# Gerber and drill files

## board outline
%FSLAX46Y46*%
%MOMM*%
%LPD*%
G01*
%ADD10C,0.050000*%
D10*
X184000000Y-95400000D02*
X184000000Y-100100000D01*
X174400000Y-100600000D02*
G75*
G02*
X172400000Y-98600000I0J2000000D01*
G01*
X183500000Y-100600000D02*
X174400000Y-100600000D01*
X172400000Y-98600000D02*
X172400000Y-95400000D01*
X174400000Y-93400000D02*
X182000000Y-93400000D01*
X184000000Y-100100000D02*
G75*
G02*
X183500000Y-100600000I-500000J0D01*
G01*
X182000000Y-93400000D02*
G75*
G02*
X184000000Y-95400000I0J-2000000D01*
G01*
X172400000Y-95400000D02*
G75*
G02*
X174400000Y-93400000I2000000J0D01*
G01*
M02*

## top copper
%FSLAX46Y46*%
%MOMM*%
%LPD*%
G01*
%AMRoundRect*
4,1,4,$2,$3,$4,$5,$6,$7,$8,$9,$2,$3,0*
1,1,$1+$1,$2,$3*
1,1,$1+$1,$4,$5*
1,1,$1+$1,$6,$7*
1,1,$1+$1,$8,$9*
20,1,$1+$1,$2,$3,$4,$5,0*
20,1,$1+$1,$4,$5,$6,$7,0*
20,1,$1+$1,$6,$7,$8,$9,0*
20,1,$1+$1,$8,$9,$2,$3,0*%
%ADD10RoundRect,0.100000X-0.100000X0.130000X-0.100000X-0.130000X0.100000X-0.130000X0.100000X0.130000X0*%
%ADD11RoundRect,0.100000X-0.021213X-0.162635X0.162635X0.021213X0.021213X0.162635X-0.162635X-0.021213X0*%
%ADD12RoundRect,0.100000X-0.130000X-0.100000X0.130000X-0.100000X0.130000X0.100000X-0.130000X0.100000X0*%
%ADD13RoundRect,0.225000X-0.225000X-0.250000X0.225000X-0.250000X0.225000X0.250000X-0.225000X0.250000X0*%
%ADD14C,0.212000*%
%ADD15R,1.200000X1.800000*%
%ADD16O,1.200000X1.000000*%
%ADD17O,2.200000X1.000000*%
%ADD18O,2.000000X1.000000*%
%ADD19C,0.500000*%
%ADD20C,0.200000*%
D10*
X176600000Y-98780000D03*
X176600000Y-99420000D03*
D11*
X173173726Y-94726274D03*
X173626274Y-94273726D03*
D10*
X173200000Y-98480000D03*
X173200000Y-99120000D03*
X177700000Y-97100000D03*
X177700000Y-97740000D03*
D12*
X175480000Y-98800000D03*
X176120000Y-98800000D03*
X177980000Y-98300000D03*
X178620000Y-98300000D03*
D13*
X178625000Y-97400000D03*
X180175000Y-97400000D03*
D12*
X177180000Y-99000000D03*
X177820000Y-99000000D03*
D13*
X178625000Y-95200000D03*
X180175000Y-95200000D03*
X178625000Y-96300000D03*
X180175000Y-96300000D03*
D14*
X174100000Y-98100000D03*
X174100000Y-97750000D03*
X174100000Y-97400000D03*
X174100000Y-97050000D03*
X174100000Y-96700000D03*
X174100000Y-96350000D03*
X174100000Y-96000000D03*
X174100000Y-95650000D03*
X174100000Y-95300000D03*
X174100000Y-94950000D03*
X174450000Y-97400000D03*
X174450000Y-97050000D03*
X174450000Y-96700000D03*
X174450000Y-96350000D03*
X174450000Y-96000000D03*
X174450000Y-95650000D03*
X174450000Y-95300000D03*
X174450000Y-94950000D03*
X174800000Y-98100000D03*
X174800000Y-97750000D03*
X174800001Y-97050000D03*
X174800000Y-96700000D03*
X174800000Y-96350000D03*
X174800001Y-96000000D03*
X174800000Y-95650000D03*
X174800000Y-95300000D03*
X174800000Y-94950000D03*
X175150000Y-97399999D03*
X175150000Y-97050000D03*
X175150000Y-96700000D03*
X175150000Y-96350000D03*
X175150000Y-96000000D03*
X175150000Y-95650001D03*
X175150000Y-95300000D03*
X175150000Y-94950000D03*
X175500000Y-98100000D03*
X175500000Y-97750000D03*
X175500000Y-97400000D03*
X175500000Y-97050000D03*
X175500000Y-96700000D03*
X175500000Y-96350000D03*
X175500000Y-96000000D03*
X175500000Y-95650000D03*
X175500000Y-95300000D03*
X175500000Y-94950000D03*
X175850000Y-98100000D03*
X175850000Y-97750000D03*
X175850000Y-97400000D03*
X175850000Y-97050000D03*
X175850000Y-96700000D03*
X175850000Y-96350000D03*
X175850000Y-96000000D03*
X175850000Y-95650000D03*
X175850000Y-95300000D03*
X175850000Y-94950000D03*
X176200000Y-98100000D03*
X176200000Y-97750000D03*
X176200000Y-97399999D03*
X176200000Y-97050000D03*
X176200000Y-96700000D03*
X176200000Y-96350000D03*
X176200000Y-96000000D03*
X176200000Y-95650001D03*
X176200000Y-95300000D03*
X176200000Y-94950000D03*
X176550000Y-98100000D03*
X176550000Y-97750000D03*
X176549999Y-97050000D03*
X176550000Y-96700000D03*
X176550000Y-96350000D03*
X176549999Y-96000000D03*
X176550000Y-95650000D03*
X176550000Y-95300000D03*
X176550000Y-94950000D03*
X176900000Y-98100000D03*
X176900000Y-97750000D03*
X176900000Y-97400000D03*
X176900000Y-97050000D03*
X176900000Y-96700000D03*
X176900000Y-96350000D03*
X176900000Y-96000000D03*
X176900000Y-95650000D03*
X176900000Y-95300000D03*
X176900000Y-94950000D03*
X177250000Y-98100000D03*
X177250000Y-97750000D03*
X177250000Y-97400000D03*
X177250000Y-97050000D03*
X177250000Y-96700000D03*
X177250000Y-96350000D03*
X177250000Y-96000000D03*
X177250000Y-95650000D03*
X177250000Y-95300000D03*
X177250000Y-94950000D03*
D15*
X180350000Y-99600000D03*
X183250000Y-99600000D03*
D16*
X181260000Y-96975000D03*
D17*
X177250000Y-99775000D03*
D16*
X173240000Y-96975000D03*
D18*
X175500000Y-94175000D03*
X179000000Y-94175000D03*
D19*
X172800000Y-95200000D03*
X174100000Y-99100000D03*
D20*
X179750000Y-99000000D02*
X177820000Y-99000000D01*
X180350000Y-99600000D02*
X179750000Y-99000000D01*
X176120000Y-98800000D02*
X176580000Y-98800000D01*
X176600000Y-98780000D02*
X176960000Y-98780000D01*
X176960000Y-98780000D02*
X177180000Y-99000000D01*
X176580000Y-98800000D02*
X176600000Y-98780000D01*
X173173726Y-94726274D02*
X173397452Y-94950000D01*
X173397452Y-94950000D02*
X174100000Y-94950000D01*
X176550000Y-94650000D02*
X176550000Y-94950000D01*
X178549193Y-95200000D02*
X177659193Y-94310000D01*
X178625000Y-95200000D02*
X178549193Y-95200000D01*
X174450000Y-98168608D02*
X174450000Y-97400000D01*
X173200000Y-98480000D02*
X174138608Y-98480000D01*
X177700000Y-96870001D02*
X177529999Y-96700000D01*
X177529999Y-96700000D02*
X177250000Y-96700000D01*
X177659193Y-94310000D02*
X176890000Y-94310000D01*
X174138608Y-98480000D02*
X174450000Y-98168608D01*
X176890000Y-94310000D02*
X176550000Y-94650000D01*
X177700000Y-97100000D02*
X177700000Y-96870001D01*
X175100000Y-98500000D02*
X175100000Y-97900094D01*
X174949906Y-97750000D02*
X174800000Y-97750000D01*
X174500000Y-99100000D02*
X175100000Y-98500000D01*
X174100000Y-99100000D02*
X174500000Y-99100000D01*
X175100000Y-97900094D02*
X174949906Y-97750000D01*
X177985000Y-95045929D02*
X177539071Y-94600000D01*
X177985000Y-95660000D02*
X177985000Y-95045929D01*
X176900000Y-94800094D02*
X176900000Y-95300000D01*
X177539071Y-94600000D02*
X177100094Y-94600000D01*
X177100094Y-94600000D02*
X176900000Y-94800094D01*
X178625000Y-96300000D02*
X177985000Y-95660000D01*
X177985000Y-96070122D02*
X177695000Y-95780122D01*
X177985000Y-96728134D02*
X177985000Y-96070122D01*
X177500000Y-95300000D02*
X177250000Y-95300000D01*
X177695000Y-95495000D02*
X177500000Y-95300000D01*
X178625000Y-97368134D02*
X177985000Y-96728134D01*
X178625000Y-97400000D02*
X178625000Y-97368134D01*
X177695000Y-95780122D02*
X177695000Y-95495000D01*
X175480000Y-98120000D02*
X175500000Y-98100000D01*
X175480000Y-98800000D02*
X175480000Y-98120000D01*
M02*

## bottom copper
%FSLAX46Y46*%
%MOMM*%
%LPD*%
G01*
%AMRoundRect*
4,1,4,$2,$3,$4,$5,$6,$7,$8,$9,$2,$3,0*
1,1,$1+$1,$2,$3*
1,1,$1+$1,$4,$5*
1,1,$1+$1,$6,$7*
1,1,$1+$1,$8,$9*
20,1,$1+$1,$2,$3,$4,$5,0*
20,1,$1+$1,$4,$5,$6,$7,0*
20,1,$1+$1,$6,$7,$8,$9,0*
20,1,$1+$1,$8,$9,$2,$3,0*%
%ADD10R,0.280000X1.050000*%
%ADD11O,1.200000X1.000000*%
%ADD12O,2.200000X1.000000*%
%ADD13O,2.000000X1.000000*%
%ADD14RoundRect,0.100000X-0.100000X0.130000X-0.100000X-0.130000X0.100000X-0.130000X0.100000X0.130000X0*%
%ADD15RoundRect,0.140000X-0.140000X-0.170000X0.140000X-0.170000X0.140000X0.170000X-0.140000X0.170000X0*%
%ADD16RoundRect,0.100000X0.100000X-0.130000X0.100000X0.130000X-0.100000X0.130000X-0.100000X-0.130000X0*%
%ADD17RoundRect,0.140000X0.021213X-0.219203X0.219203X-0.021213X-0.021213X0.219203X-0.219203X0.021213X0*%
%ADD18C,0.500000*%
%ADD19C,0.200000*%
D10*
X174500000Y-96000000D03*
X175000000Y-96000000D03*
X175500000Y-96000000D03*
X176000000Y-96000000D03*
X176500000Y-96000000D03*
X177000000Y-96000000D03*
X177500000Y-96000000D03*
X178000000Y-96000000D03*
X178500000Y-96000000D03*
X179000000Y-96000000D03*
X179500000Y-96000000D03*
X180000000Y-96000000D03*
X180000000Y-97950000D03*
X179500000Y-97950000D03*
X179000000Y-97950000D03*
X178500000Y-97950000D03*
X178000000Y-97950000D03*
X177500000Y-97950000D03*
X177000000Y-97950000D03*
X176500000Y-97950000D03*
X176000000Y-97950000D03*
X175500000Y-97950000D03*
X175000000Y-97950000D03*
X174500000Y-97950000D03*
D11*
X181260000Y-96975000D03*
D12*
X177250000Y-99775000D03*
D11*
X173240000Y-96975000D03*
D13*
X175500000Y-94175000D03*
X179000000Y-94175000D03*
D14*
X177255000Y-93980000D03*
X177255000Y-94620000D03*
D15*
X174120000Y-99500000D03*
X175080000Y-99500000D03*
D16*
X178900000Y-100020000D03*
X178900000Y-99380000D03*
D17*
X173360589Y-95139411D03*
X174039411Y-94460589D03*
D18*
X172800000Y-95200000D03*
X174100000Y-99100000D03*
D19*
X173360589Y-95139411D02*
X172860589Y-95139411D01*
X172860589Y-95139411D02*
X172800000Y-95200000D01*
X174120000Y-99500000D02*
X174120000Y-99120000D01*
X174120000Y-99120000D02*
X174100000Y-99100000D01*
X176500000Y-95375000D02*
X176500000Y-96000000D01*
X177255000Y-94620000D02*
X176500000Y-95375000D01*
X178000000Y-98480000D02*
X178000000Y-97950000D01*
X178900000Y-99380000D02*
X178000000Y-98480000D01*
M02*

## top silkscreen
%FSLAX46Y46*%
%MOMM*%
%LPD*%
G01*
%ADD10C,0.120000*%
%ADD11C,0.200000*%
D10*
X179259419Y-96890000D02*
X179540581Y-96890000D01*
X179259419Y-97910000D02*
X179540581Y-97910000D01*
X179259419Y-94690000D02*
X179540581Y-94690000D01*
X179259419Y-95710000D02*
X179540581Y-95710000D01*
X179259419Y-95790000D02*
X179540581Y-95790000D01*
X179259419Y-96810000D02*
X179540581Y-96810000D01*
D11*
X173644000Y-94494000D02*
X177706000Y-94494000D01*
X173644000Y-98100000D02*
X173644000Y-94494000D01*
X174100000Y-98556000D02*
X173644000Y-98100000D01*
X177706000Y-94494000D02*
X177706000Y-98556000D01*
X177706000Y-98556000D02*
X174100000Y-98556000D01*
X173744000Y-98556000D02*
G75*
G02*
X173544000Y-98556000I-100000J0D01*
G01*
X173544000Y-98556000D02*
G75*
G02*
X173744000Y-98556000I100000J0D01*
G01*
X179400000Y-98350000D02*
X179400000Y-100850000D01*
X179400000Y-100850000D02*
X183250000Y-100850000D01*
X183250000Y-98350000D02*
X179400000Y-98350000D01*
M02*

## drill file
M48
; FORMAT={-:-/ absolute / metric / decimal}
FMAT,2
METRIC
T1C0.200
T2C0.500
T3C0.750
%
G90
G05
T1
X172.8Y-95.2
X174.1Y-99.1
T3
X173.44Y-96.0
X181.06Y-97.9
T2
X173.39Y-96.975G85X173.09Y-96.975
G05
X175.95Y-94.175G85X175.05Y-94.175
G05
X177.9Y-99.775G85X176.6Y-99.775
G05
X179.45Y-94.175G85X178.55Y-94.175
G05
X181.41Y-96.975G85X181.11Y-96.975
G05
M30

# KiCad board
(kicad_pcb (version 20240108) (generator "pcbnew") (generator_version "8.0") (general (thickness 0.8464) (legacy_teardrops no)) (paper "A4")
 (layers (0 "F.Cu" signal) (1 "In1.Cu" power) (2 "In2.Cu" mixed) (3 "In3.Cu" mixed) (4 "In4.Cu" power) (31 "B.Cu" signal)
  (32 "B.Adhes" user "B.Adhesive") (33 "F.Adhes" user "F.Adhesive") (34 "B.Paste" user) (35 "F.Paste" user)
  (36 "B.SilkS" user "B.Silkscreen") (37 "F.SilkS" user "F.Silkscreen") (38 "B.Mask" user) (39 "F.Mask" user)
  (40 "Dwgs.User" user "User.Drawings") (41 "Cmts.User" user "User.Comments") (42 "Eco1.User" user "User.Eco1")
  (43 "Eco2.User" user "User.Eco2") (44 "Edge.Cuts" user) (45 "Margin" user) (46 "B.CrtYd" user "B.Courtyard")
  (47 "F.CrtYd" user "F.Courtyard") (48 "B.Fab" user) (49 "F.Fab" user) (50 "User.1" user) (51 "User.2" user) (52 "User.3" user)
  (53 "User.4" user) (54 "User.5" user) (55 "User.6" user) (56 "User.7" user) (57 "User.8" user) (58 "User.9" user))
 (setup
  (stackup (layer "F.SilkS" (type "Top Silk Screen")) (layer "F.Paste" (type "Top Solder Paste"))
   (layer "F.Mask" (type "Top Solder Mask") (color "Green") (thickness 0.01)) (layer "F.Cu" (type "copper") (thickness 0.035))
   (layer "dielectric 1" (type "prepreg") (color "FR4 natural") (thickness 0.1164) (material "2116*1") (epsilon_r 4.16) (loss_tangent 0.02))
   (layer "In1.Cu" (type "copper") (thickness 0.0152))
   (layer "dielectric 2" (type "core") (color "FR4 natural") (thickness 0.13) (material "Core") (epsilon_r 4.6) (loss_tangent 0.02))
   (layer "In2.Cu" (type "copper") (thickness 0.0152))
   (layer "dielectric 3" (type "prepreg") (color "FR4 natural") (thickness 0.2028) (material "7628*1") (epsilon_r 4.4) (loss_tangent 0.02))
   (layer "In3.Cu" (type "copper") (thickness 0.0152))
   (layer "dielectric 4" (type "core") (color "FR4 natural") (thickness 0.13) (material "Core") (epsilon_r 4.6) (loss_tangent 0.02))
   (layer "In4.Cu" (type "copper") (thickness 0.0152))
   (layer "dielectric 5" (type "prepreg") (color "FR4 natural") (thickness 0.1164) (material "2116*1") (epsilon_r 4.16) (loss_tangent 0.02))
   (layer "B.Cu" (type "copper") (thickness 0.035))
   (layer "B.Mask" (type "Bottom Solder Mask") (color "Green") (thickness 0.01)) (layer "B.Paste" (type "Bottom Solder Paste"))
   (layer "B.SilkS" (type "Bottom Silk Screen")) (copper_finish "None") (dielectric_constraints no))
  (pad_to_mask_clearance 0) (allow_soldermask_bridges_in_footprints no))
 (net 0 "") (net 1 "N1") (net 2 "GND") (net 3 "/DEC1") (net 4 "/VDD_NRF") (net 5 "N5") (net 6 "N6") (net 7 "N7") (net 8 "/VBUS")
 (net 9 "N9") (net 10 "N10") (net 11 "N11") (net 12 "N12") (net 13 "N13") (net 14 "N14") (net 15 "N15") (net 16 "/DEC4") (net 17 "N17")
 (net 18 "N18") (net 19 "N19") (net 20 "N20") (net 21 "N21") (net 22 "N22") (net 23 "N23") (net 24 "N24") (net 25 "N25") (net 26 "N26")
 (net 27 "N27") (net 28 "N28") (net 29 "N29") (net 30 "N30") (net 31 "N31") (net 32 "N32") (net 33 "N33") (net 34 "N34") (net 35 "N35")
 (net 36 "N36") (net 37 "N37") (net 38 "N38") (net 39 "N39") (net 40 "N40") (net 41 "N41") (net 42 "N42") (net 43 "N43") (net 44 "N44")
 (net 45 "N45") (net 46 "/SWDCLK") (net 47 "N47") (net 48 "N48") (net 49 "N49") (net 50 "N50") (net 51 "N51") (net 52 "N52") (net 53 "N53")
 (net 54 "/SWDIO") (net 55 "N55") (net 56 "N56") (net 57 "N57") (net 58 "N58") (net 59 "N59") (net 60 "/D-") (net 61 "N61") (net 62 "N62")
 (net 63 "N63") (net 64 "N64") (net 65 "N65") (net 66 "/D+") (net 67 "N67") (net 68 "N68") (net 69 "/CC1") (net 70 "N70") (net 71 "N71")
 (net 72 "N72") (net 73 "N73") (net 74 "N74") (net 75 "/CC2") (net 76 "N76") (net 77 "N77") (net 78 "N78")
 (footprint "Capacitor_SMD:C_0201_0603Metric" (layer "F.Cu") (at 176.6 99.1 -90)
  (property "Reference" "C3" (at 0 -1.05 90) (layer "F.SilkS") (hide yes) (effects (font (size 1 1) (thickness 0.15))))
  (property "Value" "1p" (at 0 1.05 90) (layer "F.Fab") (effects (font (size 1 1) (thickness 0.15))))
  (pad "" smd roundrect (at -0.345 0 270) (size 0.318 0.36) (layers "F.Paste") (roundrect_rratio 0.25))
  (pad "" smd roundrect (at 0.345 0 270) (size 0.318 0.36) (layers "F.Paste") (roundrect_rratio 0.25))
  (pad "1" smd roundrect (at -0.32 0 270) (size 0.46 0.4) (layers "F.Cu" "F.Mask") (roundrect_rratio 0.25) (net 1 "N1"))
  (pad "2" smd roundrect (at 0.32 0 270) (size 0.46 0.4) (layers "F.Cu" "F.Mask") (roundrect_rratio 0.25) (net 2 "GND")))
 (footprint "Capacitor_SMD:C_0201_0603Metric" (layer "F.Cu") (at 173.4 94.5 45)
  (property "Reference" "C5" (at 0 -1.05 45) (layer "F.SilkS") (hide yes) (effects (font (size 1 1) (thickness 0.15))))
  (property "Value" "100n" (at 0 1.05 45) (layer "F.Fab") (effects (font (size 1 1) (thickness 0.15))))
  (pad "" smd roundrect (at -0.345 0 45) (size 0.318 0.36) (layers "F.Paste") (roundrect_rratio 0.25))
  (pad "" smd roundrect (at 0.345 0 45) (size 0.318 0.36) (layers "F.Paste") (roundrect_rratio 0.25))
  (pad "1" smd roundrect (at -0.32 0 45) (size 0.46 0.4) (layers "F.Cu" "F.Mask") (roundrect_rratio 0.25) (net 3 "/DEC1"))
  (pad "2" smd roundrect (at 0.32 0 45) (size 0.46 0.4) (layers "F.Cu" "F.Mask") (roundrect_rratio 0.25) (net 2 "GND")))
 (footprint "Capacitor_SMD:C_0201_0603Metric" (layer "F.Cu") (at 173.2 98.8 -90)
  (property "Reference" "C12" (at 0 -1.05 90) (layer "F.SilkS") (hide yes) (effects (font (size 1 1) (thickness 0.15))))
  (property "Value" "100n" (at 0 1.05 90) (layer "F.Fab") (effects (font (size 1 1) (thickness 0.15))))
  (pad "" smd roundrect (at -0.345 0 270) (size 0.318 0.36) (layers "F.Paste") (roundrect_rratio 0.25))
  (pad "" smd roundrect (at 0.345 0 270) (size 0.318 0.36) (layers "F.Paste") (roundrect_rratio 0.25))
  (pad "1" smd roundrect (at -0.32 0 270) (size 0.46 0.4) (layers "F.Cu" "F.Mask") (roundrect_rratio 0.25) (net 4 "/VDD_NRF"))
  (pad "2" smd roundrect (at 0.32 0 270) (size 0.46 0.4) (layers "F.Cu" "F.Mask") (roundrect_rratio 0.25) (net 2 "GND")))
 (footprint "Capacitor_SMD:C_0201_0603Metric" (layer "F.Cu") (at 177.7 97.42 -90)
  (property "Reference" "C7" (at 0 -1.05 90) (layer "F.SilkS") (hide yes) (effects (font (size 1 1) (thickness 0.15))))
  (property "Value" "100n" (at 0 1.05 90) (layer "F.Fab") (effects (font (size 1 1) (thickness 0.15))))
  (pad "" smd roundrect (at -0.345 0 270) (size 0.318 0.36) (layers "F.Paste") (roundrect_rratio 0.25))
  (pad "" smd roundrect (at 0.345 0 270) (size 0.318 0.36) (layers "F.Paste") (roundrect_rratio 0.25))
  (pad "1" smd roundrect (at -0.32 0 270) (size 0.46 0.4) (layers "F.Cu" "F.Mask") (roundrect_rratio 0.25) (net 4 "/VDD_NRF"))
  (pad "2" smd roundrect (at 0.32 0 270) (size 0.46 0.4) (layers "F.Cu" "F.Mask") (roundrect_rratio 0.25) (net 2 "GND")))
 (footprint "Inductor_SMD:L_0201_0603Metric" (layer "F.Cu") (at 175.8 98.8)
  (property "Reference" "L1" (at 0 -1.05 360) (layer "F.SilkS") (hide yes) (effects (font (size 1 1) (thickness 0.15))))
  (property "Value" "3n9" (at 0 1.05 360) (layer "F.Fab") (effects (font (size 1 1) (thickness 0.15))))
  (pad "" smd roundrect (at -0.345 0) (size 0.318 0.36) (layers "F.Paste") (roundrect_rratio 0.25))
  (pad "" smd roundrect (at 0.345 0) (size 0.318 0.36) (layers "F.Paste") (roundrect_rratio 0.25))
  (pad "1" smd roundrect (at -0.32 0) (size 0.46 0.4) (layers "F.Cu" "F.Mask") (roundrect_rratio 0.25) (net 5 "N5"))
  (pad "2" smd roundrect (at 0.32 0) (size 0.46 0.4) (layers "F.Cu" "F.Mask") (roundrect_rratio 0.25) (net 1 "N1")))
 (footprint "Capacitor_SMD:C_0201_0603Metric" (layer "F.Cu") (at 178.3 98.3)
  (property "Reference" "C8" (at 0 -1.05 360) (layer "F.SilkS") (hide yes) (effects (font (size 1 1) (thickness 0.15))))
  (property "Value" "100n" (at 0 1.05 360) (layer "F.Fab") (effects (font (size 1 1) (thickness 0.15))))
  (pad "" smd roundrect (at -0.345 0) (size 0.318 0.36) (layers "F.Paste") (roundrect_rratio 0.25))
  (pad "" smd roundrect (at 0.345 0) (size 0.318 0.36) (layers "F.Paste") (roundrect_rratio 0.25))
  (pad "1" smd roundrect (at -0.32 0) (size 0.46 0.4) (layers "F.Cu" "F.Mask") (roundrect_rratio 0.25) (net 4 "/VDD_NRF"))
  (pad "2" smd roundrect (at 0.32 0) (size 0.46 0.4) (layers "F.Cu" "F.Mask") (roundrect_rratio 0.25) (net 2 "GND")))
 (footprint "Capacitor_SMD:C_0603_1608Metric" (layer "F.Cu") (at 179.4 97.4)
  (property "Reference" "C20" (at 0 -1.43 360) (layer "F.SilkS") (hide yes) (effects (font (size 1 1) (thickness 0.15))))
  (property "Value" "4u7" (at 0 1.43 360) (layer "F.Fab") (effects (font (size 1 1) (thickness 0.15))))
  (fp_line (start -0.140581 -0.51) (end 0.140581 -0.51) (stroke (width 0.12) (type solid)) (layer "F.SilkS"))
  (fp_line (start -0.140581 0.51) (end 0.140581 0.51) (stroke (width 0.12) (type solid)) (layer "F.SilkS"))
  (pad "1" smd roundrect (at -0.775 0) (size 0.9 0.95) (layers "F.Cu" "F.Paste" "F.Mask") (roundrect_rratio 0.25) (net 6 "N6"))
  (pad "2" smd roundrect (at 0.775 0) (size 0.9 0.95) (layers "F.Cu" "F.Paste" "F.Mask") (roundrect_rratio 0.25) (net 2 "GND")))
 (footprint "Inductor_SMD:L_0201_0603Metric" (layer "F.Cu") (at 177.5 99)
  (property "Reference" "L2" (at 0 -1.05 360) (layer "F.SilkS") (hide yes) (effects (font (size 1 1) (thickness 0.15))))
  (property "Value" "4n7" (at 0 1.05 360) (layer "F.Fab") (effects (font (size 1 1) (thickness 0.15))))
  (pad "" smd roundrect (at -0.345 0) (size 0.318 0.36) (layers "F.Paste") (roundrect_rratio 0.25))
  (pad "" smd roundrect (at 0.345 0) (size 0.318 0.36) (layers "F.Paste") (roundrect_rratio 0.25))
  (pad "1" smd roundrect (at -0.32 0) (size 0.46 0.4) (layers "F.Cu" "F.Mask") (roundrect_rratio 0.25) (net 1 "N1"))
  (pad "2" smd roundrect (at 0.32 0) (size 0.46 0.4) (layers "F.Cu" "F.Mask") (roundrect_rratio 0.25) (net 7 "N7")))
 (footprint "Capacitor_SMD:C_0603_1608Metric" (layer "F.Cu") (at 179.4 95.2)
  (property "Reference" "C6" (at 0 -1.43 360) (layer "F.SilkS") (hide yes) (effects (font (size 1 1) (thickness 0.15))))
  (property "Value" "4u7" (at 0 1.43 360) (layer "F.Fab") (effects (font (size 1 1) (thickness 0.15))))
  (fp_line (start -0.140581 -0.51) (end 0.140581 -0.51) (stroke (width 0.12) (type solid)) (layer "F.SilkS"))
  (fp_line (start -0.140581 0.51) (end 0.140581 0.51) (stroke (width 0.12) (type solid)) (layer "F.SilkS"))
  (pad "1" smd roundrect (at -0.775 0) (size 0.9 0.95) (layers "F.Cu" "F.Paste" "F.Mask") (roundrect_rratio 0.25) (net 4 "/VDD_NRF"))
  (pad "2" smd roundrect (at 0.775 0) (size 0.9 0.95) (layers "F.Cu" "F.Paste" "F.Mask") (roundrect_rratio 0.25) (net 2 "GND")))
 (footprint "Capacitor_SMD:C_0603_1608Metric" (layer "F.Cu") (at 179.4 96.3)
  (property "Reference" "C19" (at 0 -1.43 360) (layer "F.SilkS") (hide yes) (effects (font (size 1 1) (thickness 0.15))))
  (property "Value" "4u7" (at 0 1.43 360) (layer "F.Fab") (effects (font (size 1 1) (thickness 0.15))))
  (fp_line (start -0.140581 -0.51) (end 0.140581 -0.51) (stroke (width 0.12) (type solid)) (layer "F.SilkS"))
  (fp_line (start -0.140581 0.51) (end 0.140581 0.51) (stroke (width 0.12) (type solid)) (layer "F.SilkS"))
  (pad "1" smd roundrect (at -0.775 0) (size 0.9 0.95) (layers "F.Cu" "F.Paste" "F.Mask") (roundrect_rratio 0.25) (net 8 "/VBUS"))
  (pad "2" smd roundrect (at 0.775 0) (size 0.9 0.95) (layers "F.Cu" "F.Paste" "F.Mask") (roundrect_rratio 0.25) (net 2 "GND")))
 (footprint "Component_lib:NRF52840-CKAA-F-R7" (layer "F.Cu") (at 175.675 96.525 90)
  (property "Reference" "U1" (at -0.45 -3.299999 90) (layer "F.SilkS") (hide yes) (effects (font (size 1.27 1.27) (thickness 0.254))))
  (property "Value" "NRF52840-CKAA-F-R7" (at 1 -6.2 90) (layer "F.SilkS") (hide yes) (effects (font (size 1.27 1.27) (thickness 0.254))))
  (fp_line (start 2.031 -2.031) (end 2.031 2.031) (stroke (width 0.2) (type solid)) (layer "F.SilkS"))
  (fp_line (start -1.575 -2.031) (end 2.031 -2.031) (stroke (width 0.2) (type solid)) (layer "F.SilkS"))
  (fp_line (start -2.031 -1.575) (end -1.575 -2.031) (stroke (width 0.2) (type solid)) (layer "F.SilkS"))
  (fp_line (start 2.031 2.031) (end -2.031 2.031) (stroke (width 0.2) (type solid)) (layer "F.SilkS"))
  (fp_line (start -2.031 2.031) (end -2.031 -1.575) (stroke (width 0.2) (type solid)) (layer "F.SilkS"))
  (fp_circle (center -2.031 -2.031) (end -2.031 -1.931) (stroke (width 0.2) (type solid)) (fill none) (layer "F.SilkS"))
  (pad "A1" smd circle (at -1.575 -1.575 180) (size 0.212 0.212) (layers "F.Cu" "F.Paste" "F.Mask") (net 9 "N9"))
  (pad "A2" smd circle (at -1.225 -1.575 180) (size 0.212 0.212) (layers "F.Cu" "F.Paste" "F.Mask") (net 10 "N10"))
  (pad "A3" smd circle (at -0.875 -1.575 180) (size 0.212 0.212) (layers "F.Cu" "F.Paste" "F.Mask") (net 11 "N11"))
  (pad "A4" smd circle (at -0.525 -1.575 180) (size 0.212 0.212) (layers "F.Cu" "F.Paste" "F.Mask") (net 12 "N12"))
  (pad "A5" smd circle (at -0.175 -1.575 180) (size 0.212 0.212) (layers "F.Cu" "F.Paste" "F.Mask") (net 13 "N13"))
  (pad "A6" smd circle (at 0.175 -1.575 180) (size 0.212 0.212) (layers "F.Cu" "F.Paste" "F.Mask") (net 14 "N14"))
  (pad "A7" smd circle (at 0.525 -1.575 180) (size 0.212 0.212) (layers "F.Cu" "F.Paste" "F.Mask") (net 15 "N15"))
  (pad "A8" smd circle (at 0.875 -1.575 180) (size 0.212 0.212) (layers "F.Cu" "F.Paste" "F.Mask") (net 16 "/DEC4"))
  (pad "A9" smd circle (at 1.225 -1.575 180) (size 0.212 0.212) (layers "F.Cu" "F.Paste" "F.Mask") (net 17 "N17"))
  (pad "A10" smd circle (at 1.575 -1.575 180) (size 0.212 0.212) (layers "F.Cu" "F.Paste" "F.Mask") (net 3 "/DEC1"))
  (pad "B3" smd circle (at -0.875 -1.225 180) (size 0.212 0.212) (layers "F.Cu" "F.Paste" "F.Mask") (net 4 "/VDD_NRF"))
  (pad "B4" smd circle (at -0.525 -1.225 180) (size 0.212 0.212) (layers "F.Cu" "F.Paste" "F.Mask") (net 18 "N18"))
  (pad "B5" smd circle (at -0.175 -1.225 180) (size 0.212 0.212) (layers "F.Cu" "F.Paste" "F.Mask") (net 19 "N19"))
  (pad "B6" smd circle (at 0.175 -1.225 180) (size 0.212 0.212) (layers "F.Cu" "F.Paste" "F.Mask") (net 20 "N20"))
  (pad "B7" smd circle (at 0.525 -1.225 180) (size 0.212 0.212) (layers "F.Cu" "F.Paste" "F.Mask") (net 2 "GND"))
  (pad "B8" smd circle (at 0.875 -1.225 180) (size 0.212 0.212) (layers "F.Cu" "F.Paste" "F.Mask") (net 4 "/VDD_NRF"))
  (pad "B9" smd circle (at 1.225 -1.225 180) (size 0.212 0.212) (layers "F.Cu" "F.Paste" "F.Mask") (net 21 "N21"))
  (pad "B10" smd circle (at 1.575 -1.225 180) (size 0.212 0.212) (layers "F.Cu" "F.Paste" "F.Mask") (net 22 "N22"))
  (pad "C1" smd circle (at -1.575 -0.875 180) (size 0.212 0.212) (layers "F.Cu" "F.Paste" "F.Mask") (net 2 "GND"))
  (pad "C2" smd circle (at -1.225 -0.875 180) (size 0.212 0.212) (layers "F.Cu" "F.Paste" "F.Mask") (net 16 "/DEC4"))
  (pad "C4" smd circle (at -0.525 -0.874999 180) (size 0.212 0.212) (layers "F.Cu" "F.Paste" "F.Mask") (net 2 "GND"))
  (pad "C5" smd circle (at -0.175 -0.875 180) (size 0.212 0.212) (layers "F.Cu" "F.Paste" "F.Mask") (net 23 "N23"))
  (pad "C6" smd circle (at 0.175 -0.875 180) (size 0.212 0.212) (layers "F.Cu" "F.Paste" "F.Mask") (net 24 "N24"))
  (pad "C7" smd circle (at 0.525 -0.874999 180) (size 0.212 0.212) (layers "F.Cu" "F.Paste" "F.Mask") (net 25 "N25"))
  (pad "C8" smd circle (at 0.875 -0.875 180) (size 0.212 0.212) (layers "F.Cu" "F.Paste" "F.Mask") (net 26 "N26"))
  (pad "C9" smd circle (at 1.225 -0.875 180) (size 0.212 0.212) (layers "F.Cu" "F.Paste" "F.Mask") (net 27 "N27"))
  (pad "C10" smd circle (at 1.575 -0.875 180) (size 0.212 0.212) (layers "F.Cu" "F.Paste" "F.Mask") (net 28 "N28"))
  (pad "D3" smd circle (at -0.874999 -0.525 180) (size 0.212 0.212) (layers "F.Cu" "F.Paste" "F.Mask") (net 2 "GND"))
  (pad "D4" smd circle (at -0.525 -0.525 180) (size 0.212 0.212) (layers "F.Cu" "F.Paste" "F.Mask") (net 2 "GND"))
  (pad "D5" smd circle (at -0.175 -0.525 180) (size 0.212 0.212) (layers "F.Cu" "F.Paste" "F.Mask") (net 2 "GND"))
  (pad "D6" smd circle (at 0.175 -0.525 180) (size 0.212 0.212) (layers "F.Cu" "F.Paste" "F.Mask") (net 2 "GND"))
  (pad "D7" smd circle (at 0.525 -0.525 180) (size 0.212 0.212) (layers "F.Cu" "F.Paste" "F.Mask") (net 2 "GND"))
  (pad "D8" smd circle (at 0.874999 -0.525 180) (size 0.212 0.212) (layers "F.Cu" "F.Paste" "F.Mask") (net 2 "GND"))
  (pad "D9" smd circle (at 1.225 -0.525 180) (size 0.212 0.212) (layers "F.Cu" "F.Paste" "F.Mask") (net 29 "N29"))
  (pad "D10" smd circle (at 1.575 -0.525 180) (size 0.212 0.212) (layers "F.Cu" "F.Paste" "F.Mask") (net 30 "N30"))
  (pad "E1" smd circle (at -1.575 -0.175 180) (size 0.212 0.212) (layers "F.Cu" "F.Paste" "F.Mask") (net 5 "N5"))
  (pad "E2" smd circle (at -1.225 -0.175 180) (size 0.212 0.212) (layers "F.Cu" "F.Paste" "F.Mask") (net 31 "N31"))
  (pad "E3" smd circle (at -0.875 -0.175 180) (size 0.212 0.212) (layers "F.Cu" "F.Paste" "F.Mask") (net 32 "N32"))
  (pad "E4" smd circle (at -0.525 -0.175 180) (size 0.212 0.212) (layers "F.Cu" "F.Paste" "F.Mask") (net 2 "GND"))
  (pad "E5" smd circle (at -0.175 -0.175 180) (size 0.212 0.212) (layers "F.Cu" "F.Paste" "F.Mask") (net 2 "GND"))
  (pad "E6" smd circle (at 0.175 -0.175 180) (size 0.212 0.212) (layers "F.Cu" "F.Paste" "F.Mask") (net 2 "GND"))
  (pad "E7" smd circle (at 0.525 -0.175 180) (size 0.212 0.212) (layers "F.Cu" "F.Paste" "F.Mask") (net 2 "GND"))
  (pad "E8" smd circle (at 0.875 -0.175 180) (size 0.212 0.212) (layers "F.Cu" "F.Paste" "F.Mask") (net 2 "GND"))
  (pad "E9" smd circle (at 1.225 -0.175 180) (size 0.212 0.212) (layers "F.Cu" "F.Paste" "F.Mask") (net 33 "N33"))
  (pad "E10" smd circle (at 1.575 -0.175 180) (size 0.212 0.212) (layers "F.Cu" "F.Paste" "F.Mask") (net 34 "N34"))
  (pad "F1" smd circle (at -1.575 0.175 180) (size 0.212 0.212) (layers "F.Cu" "F.Paste" "F.Mask") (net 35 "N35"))
  (pad "F2" smd circle (at -1.225 0.175 180) (size 0.212 0.212) (layers "F.Cu" "F.Paste" "F.Mask") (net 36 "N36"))
  (pad "F3" smd circle (at -0.875 0.175 180) (size 0.212 0.212) (layers "F.Cu" "F.Paste" "F.Mask") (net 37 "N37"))
  (pad "F4" smd circle (at -0.525 0.175 180) (size 0.212 0.212) (layers "F.Cu" "F.Paste" "F.Mask") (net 2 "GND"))
  (pad "F5" smd circle (at -0.175 0.175 180) (size 0.212 0.212) (layers "F.Cu" "F.Paste" "F.Mask") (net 2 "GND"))
  (pad "F6" smd circle (at 0.175 0.175 180) (size 0.212 0.212) (layers "F.Cu" "F.Paste" "F.Mask") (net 2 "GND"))
  (pad "F7" smd circle (at 0.525 0.175 180) (size 0.212 0.212) (layers "F.Cu" "F.Paste" "F.Mask") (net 2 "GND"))
  (pad "F8" smd circle (at 0.875 0.175 180) (size 0.212 0.212) (layers "F.Cu" "F.Paste" "F.Mask") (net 2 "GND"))
  (pad "F9" smd circle (at 1.225 0.175 180) (size 0.212 0.212) (layers "F.Cu" "F.Paste" "F.Mask") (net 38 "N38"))
  (pad "F10" smd circle (at 1.575 0.175 180) (size 0.212 0.212) (layers "F.Cu" "F.Paste" "F.Mask") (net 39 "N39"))
  (pad "G1" smd circle (at -1.575 0.525 180) (size 0.212 0.212) (layers "F.Cu" "F.Paste" "F.Mask") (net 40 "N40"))
  (pad "G2" smd circle (at -1.225 0.525 180) (size 0.212 0.212) (layers "F.Cu" "F.Paste" "F.Mask") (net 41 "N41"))
  (pad "G3" smd circle (at -0.874999 0.525 180) (size 0.212 0.212) (layers "F.Cu" "F.Paste" "F.Mask") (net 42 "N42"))
  (pad "G4" smd circle (at -0.525 0.525 180) (size 0.212 0.212) (layers "F.Cu" "F.Paste" "F.Mask") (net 2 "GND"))
  (pad "G5" smd circle (at -0.175 0.525 180) (size 0.212 0.212) (layers "F.Cu" "F.Paste" "F.Mask") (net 2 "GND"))
  (pad "G6" smd circle (at 0.175 0.525 180) (size 0.212 0.212) (layers "F.Cu" "F.Paste" "F.Mask") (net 2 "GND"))
  (pad "G7" smd circle (at 0.525 0.525 180) (size 0.212 0.212) (layers "F.Cu" "F.Paste" "F.Mask") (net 2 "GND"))
  (pad "G8" smd circle (at 0.874999 0.525 180) (size 0.212 0.212) (layers "F.Cu" "F.Paste" "F.Mask") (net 2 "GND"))
  (pad "G9" smd circle (at 1.225 0.525 180) (size 0.212 0.212) (layers "F.Cu" "F.Paste" "F.Mask") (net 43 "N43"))
  (pad "G10" smd circle (at 1.575 0.525 180) (size 0.212 0.212) (layers "F.Cu" "F.Paste" "F.Mask") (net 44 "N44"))
  (pad "H1" smd circle (at -1.575 0.875 180) (size 0.212 0.212) (layers "F.Cu" "F.Paste" "F.Mask") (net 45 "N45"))
  (pad "H2" smd circle (at -1.225 0.875 180) (size 0.212 0.212) (layers "F.Cu" "F.Paste" "F.Mask") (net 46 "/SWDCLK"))
  (pad "H4" smd circle (at -0.525 0.874999 180) (size 0.212 0.212) (layers "F.Cu" "F.Paste" "F.Mask") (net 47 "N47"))
  (pad "H5" smd circle (at -0.175 0.875 180) (size 0.212 0.212) (layers "F.Cu" "F.Paste" "F.Mask") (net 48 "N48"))
  (pad "H6" smd circle (at 0.175 0.875 180) (size 0.212 0.212) (layers "F.Cu" "F.Paste" "F.Mask") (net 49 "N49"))
  (pad "H7" smd circle (at 0.525 0.874999 180) (size 0.212 0.212) (layers "F.Cu" "F.Paste" "F.Mask") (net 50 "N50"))
  (pad "H8" smd circle (at 0.875 0.875 180) (size 0.212 0.212) (layers "F.Cu" "F.Paste" "F.Mask") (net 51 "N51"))
  (pad "H9" smd circle (at 1.225 0.875 180) (size 0.212 0.212) (layers "F.Cu" "F.Paste" "F.Mask") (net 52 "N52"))
  (pad "H10" smd circle (at 1.575 0.875 180) (size 0.212 0.212) (layers "F.Cu" "F.Paste" "F.Mask") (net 4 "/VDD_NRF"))
  (pad "J1" smd circle (at -1.575 1.225 180) (size 0.212 0.212) (layers "F.Cu" "F.Paste" "F.Mask") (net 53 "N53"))
  (pad "J2" smd circle (at -1.225 1.225 180) (size 0.212 0.212) (layers "F.Cu" "F.Paste" "F.Mask") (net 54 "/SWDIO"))
  (pad "J3" smd circle (at -0.875 1.225 180) (size 0.212 0.212) (layers "F.Cu" "F.Paste" "F.Mask") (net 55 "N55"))
  (pad "J4" smd circle (at -0.525 1.225 180) (size 0.212 0.212) (layers "F.Cu" "F.Paste" "F.Mask") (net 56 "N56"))
  (pad "J5" smd circle (at -0.175 1.225 180) (size 0.212 0.212) (layers "F.Cu" "F.Paste" "F.Mask") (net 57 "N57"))
  (pad "J6" smd circle (at 0.175 1.225 180) (size 0.212 0.212) (layers "F.Cu" "F.Paste" "F.Mask") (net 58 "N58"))
  (pad "J7" smd circle (at 0.525 1.225 180) (size 0.212 0.212) (layers "F.Cu" "F.Paste" "F.Mask") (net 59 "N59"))
  (pad "J8" smd circle (at 0.875 1.225 180) (size 0.212 0.212) (layers "F.Cu" "F.Paste" "F.Mask") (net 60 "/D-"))
  (pad "J9" smd circle (at 1.225 1.225 180) (size 0.212 0.212) (layers "F.Cu" "F.Paste" "F.Mask") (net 8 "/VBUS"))
  (pad "J10" smd circle (at 1.575 1.225 180) (size 0.212 0.212) (layers "F.Cu" "F.Paste" "F.Mask") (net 8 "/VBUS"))
  (pad "K1" smd circle (at -1.575 1.575 180) (size 0.212 0.212) (layers "F.Cu" "F.Paste" "F.Mask") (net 4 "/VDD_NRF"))
  (pad "K2" smd circle (at -1.225 1.575 180) (size 0.212 0.212) (layers "F.Cu" "F.Paste" "F.Mask") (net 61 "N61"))
  (pad "K3" smd circle (at -0.875 1.575 180) (size 0.212 0.212) (layers "F.Cu" "F.Paste" "F.Mask") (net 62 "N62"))
  (pad "K4" smd circle (at -0.525 1.575 180) (size 0.212 0.212) (layers "F.Cu" "F.Paste" "F.Mask") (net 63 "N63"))
  (pad "K5" smd circle (at -0.175 1.575 180) (size 0.212 0.212) (layers "F.Cu" "F.Paste" "F.Mask") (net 4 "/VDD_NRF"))
  (pad "K6" smd circle (at 0.175 1.575 180) (size 0.212 0.212) (layers "F.Cu" "F.Paste" "F.Mask") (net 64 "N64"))
  (pad "K7" smd circle (at 0.525 1.575 180) (size 0.212 0.212) (layers "F.Cu" "F.Paste" "F.Mask") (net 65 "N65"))
  (pad "K8" smd circle (at 0.875 1.575 180) (size 0.212 0.212) (layers "F.Cu" "F.Paste" "F.Mask") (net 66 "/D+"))
  (pad "K9" smd circle (at 1.225 1.575 180) (size 0.212 0.212) (layers "F.Cu" "F.Paste" "F.Mask") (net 6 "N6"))
  (pad "K10" smd circle (at 1.575 1.575 180) (size 0.212 0.212) (layers "F.Cu" "F.Paste" "F.Mask") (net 2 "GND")))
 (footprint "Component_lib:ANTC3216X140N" (layer "F.Cu") (at 181.8 99.6)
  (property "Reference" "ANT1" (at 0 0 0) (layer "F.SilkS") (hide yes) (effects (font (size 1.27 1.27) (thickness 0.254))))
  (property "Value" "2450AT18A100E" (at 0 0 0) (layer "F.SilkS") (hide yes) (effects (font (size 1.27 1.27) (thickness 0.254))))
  (fp_line (start -2.4 -1.25) (end -2.4 1.25) (stroke (width 0.2) (type solid)) (layer "F.SilkS"))
  (fp_line (start -2.4 1.25) (end 1.45 1.25) (stroke (width 0.2) (type solid)) (layer "F.SilkS"))
  (fp_line (start 1.45 -1.25) (end -2.4 -1.25) (stroke (width 0.2) (type solid)) (layer "F.SilkS"))
  (pad "1" smd rect (at -1.45 0) (size 1.2 1.8) (layers "F.Cu" "F.Paste" "F.Mask") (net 7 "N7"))
  (pad "2" smd rect (at 1.45 0) (size 1.2 1.8) (layers "F.Cu" "F.Paste" "F.Mask")))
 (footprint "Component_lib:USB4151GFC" (layer "B.Cu") (at 177.25 96.975 180)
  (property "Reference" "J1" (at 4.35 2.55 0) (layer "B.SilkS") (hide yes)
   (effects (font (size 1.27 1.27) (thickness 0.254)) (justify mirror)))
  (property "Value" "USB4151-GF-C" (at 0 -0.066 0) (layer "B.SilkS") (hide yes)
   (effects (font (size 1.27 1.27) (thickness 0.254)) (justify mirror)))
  (pad "" np_thru_hole circle (at -3.81 -0.925 180) (size 0.75 0.75) (drill 0.75) (layers "*.Cu" "*.Mask"))
  (pad "" np_thru_hole circle (at 3.81 0.975 180) (size 0.75 0.75) (drill 0.75) (layers "*.Cu" "*.Mask"))
  (pad "A1" smd rect (at 2.75 0.975 180) (size 0.28 1.05) (layers "B.Cu" "B.Paste" "B.Mask") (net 2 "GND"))
  (pad "A2" smd rect (at 2.25 0.975 180) (size 0.28 1.05) (layers "B.Cu" "B.Paste" "B.Mask") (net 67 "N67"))
  (pad "A3" smd rect (at 1.75 0.975 180) (size 0.28 1.05) (layers "B.Cu" "B.Paste" "B.Mask") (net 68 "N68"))
  (pad "A4" smd rect (at 1.25 0.975 180) (size 0.28 1.05) (layers "B.Cu" "B.Paste" "B.Mask") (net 8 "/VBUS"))
  (pad "A5" smd rect (at 0.75 0.975 180) (size 0.28 1.05) (layers "B.Cu" "B.Paste" "B.Mask") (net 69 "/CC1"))
  (pad "A6" smd rect (at 0.25 0.975 180) (size 0.28 1.05) (layers "B.Cu" "B.Paste" "B.Mask") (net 66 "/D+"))
  (pad "A7" smd rect (at -0.25 0.975 180) (size 0.28 1.05) (layers "B.Cu" "B.Paste" "B.Mask") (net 60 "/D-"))
  (pad "A8" smd rect (at -0.75 0.975 180) (size 0.28 1.05) (layers "B.Cu" "B.Paste" "B.Mask") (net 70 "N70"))
  (pad "A9" smd rect (at -1.25 0.975 180) (size 0.28 1.05) (layers "B.Cu" "B.Paste" "B.Mask") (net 8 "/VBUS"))
  (pad "A10" smd rect (at -1.75 0.975 180) (size 0.28 1.05) (layers "B.Cu" "B.Paste" "B.Mask") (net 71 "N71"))
  (pad "A11" smd rect (at -2.25 0.975 180) (size 0.28 1.05) (layers "B.Cu" "B.Paste" "B.Mask") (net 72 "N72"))
  (pad "A12" smd rect (at -2.75 0.975 180) (size 0.28 1.05) (layers "B.Cu" "B.Paste" "B.Mask") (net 2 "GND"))
  (pad "B1" smd rect (at -2.75 -0.975 180) (size 0.28 1.05) (layers "B.Cu" "B.Paste" "B.Mask") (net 2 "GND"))
  (pad "B2" smd rect (at -2.25 -0.975 180) (size 0.28 1.05) (layers "B.Cu" "B.Paste" "B.Mask") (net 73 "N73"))
  (pad "B3" smd rect (at -1.75 -0.975 180) (size 0.28 1.05) (layers "B.Cu" "B.Paste" "B.Mask") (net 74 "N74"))
  (pad "B4" smd rect (at -1.25 -0.975 180) (size 0.28 1.05) (layers "B.Cu" "B.Paste" "B.Mask") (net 8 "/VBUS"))
  (pad "B5" smd rect (at -0.75 -0.975 180) (size 0.28 1.05) (layers "B.Cu" "B.Paste" "B.Mask") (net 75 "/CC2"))
  (pad "B6" smd rect (at -0.25 -0.975 180) (size 0.28 1.05) (layers "B.Cu" "B.Paste" "B.Mask") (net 66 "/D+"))
  (pad "B7" smd rect (at 0.25 -0.975 180) (size 0.28 1.05) (layers "B.Cu" "B.Paste" "B.Mask") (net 60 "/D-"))
  (pad "B8" smd rect (at 0.75 -0.975 180) (size 0.28 1.05) (layers "B.Cu" "B.Paste" "B.Mask") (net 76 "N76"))
  (pad "B9" smd rect (at 1.25 -0.975 180) (size 0.28 1.05) (layers "B.Cu" "B.Paste" "B.Mask") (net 8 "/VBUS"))
  (pad "B10" smd rect (at 1.75 -0.975 180) (size 0.28 1.05) (layers "B.Cu" "B.Paste" "B.Mask") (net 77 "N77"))
  (pad "B11" smd rect (at 2.25 -0.975 180) (size 0.28 1.05) (layers "B.Cu" "B.Paste" "B.Mask") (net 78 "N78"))
  (pad "B12" smd rect (at 2.75 -0.975 180) (size 0.28 1.05) (layers "B.Cu" "B.Paste" "B.Mask") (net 2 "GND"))
  (pad "MH1" thru_hole oval (at -4.01 0 180) (size 1.2 1) (drill oval 0.8 0.5) (layers "*.Cu" "*.Mask") (remove_unused_layers no)
   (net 2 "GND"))
  (pad "MH2" thru_hole oval (at 0 -2.8 180) (size 2.2 1) (drill oval 1.8 0.5) (layers "*.Cu" "*.Mask") (remove_unused_layers no)
   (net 2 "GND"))
  (pad "MH3" thru_hole oval (at 4.01 0 180) (size 1.2 1) (drill oval 0.8 0.5) (layers "*.Cu" "*.Mask") (remove_unused_layers no)
   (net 2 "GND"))
  (pad "MH4" thru_hole oval (at 1.75 2.8 180) (size 2 1) (drill oval 1.4 0.5) (layers "*.Cu" "*.Mask") (remove_unused_layers no)
   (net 2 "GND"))
  (pad "MH5" thru_hole oval (at -1.75 2.8 180) (size 2 1) (drill oval 1.4 0.5) (layers "*.Cu" "*.Mask") (remove_unused_layers no)
   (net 2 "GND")))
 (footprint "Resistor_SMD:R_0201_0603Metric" (layer "B.Cu") (at 177.255 94.3 -90)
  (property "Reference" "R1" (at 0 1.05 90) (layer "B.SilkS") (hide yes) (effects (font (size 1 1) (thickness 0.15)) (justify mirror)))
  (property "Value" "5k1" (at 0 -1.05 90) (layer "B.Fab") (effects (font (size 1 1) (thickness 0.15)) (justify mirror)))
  (pad "" smd roundrect (at -0.345 0 270) (size 0.318 0.36) (layers "B.Paste") (roundrect_rratio 0.25))
  (pad "" smd roundrect (at 0.345 0 270) (size 0.318 0.36) (layers "B.Paste") (roundrect_rratio 0.25))
  (pad "1" smd roundrect (at -0.32 0 270) (size 0.46 0.4) (layers "B.Cu" "B.Mask") (roundrect_rratio 0.25) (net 2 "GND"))
  (pad "2" smd roundrect (at 0.32 0 270) (size 0.46 0.4) (layers "B.Cu" "B.Mask") (roundrect_rratio 0.25) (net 69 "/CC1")))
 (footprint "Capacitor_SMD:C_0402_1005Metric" (layer "B.Cu") (at 174.6 99.5)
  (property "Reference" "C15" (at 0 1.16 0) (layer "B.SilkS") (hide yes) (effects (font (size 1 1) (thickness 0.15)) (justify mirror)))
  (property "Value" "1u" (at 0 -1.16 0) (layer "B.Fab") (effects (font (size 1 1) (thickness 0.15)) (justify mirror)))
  (pad "1" smd roundrect (at -0.48 0) (size 0.56 0.62) (layers "B.Cu" "B.Paste" "B.Mask") (roundrect_rratio 0.25) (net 16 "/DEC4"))
  (pad "2" smd roundrect (at 0.48 0) (size 0.56 0.62) (layers "B.Cu" "B.Paste" "B.Mask") (roundrect_rratio 0.25) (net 2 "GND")))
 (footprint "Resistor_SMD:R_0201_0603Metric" (layer "B.Cu") (at 178.9 99.7 90)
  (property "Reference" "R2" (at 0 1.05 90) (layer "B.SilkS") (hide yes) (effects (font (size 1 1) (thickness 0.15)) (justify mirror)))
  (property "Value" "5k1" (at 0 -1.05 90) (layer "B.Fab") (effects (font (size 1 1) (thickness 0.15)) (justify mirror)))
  (pad "" smd roundrect (at -0.345 0 90) (size 0.318 0.36) (layers "B.Paste") (roundrect_rratio 0.25))
  (pad "" smd roundrect (at 0.345 0 90) (size 0.318 0.36) (layers "B.Paste") (roundrect_rratio 0.25))
  (pad "1" smd roundrect (at -0.32 0 90) (size 0.46 0.4) (layers "B.Cu" "B.Mask") (roundrect_rratio 0.25) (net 2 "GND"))
  (pad "2" smd roundrect (at 0.32 0 90) (size 0.46 0.4) (layers "B.Cu" "B.Mask") (roundrect_rratio 0.25) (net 75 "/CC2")))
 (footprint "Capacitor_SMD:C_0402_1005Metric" (layer "B.Cu") (at 173.7 94.8 45)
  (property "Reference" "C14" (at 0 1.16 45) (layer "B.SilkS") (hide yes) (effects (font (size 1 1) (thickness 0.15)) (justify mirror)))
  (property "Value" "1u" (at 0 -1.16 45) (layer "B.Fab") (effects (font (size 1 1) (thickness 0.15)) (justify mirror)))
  (pad "1" smd roundrect (at -0.48 0 45) (size 0.56 0.62) (layers "B.Cu" "B.Paste" "B.Mask") (roundrect_rratio 0.25) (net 4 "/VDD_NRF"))
  (pad "2" smd roundrect (at 0.48 0 45) (size 0.56 0.62) (layers "B.Cu" "B.Paste" "B.Mask") (roundrect_rratio 0.25) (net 2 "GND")))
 (gr_line (start 184 95.4) (end 184 100.1) (stroke (width 0.05) (type default)) (layer "Edge.Cuts"))
 (gr_arc (start 174.4 100.6) (mid 172.985786 100.014214) (end 172.4 98.6) (stroke (width 0.05) (type default)) (layer "Edge.Cuts"))
 (gr_line (start 183.5 100.6) (end 174.4 100.6) (stroke (width 0.05) (type default)) (layer "Edge.Cuts"))
 (gr_line (start 172.4 98.6) (end 172.4 95.4) (stroke (width 0.05) (type default)) (layer "Edge.Cuts"))
 (gr_line (start 174.4 93.4) (end 182 93.4) (stroke (width 0.05) (type default)) (layer "Edge.Cuts"))
 (gr_arc (start 184 100.1) (mid 183.853553 100.453553) (end 183.5 100.6) (stroke (width 0.05) (type default)) (layer "Edge.Cuts"))
 (gr_arc (start 182 93.4) (mid 183.414214 93.985786) (end 184 95.4) (stroke (width 0.05) (type default)) (layer "Edge.Cuts"))
 (gr_arc (start 172.4 95.4) (mid 172.985786 93.985786) (end 174.4 93.4) (stroke (width 0.05) (type default)) (layer "Edge.Cuts"))
 (segment (start 179.75 99) (end 177.82 99) (width 0.2) (layer "F.Cu") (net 7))
 (segment (start 180.35 99.6) (end 179.75 99) (width 0.2) (layer "F.Cu") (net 7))
 (segment (start 176.12 98.8) (end 176.58 98.8) (width 0.2) (layer "F.Cu") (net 1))
 (segment (start 176.6 98.78) (end 176.96 98.78) (width 0.2) (layer "F.Cu") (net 1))
 (segment (start 176.96 98.78) (end 177.18 99) (width 0.2) (layer "F.Cu") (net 1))
 (segment (start 176.58 98.8) (end 176.6 98.78) (width 0.2) (layer "F.Cu") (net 1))
 (segment (start 173.173726 94.726274) (end 173.397452 94.95) (width 0.2) (layer "F.Cu") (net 3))
 (segment (start 173.397452 94.95) (end 174.1 94.95) (width 0.2) (layer "F.Cu") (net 3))
 (segment (start 176.55 94.65) (end 176.55 94.95) (width 0.2) (layer "F.Cu") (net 4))
 (segment (start 178.549193 95.2) (end 177.659193 94.31) (width 0.2) (layer "F.Cu") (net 4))
 (segment (start 178.625 95.2) (end 178.549193 95.2) (width 0.2) (layer "F.Cu") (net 4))
 (segment (start 174.45 98.168608) (end 174.45 97.4) (width 0.2) (layer "F.Cu") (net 4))
 (segment (start 173.2 98.48) (end 174.138608 98.48) (width 0.2) (layer "F.Cu") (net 4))
 (segment (start 177.7 96.870001) (end 177.529999 96.7) (width 0.2) (layer "F.Cu") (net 4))
 (segment (start 177.529999 96.7) (end 177.25 96.7) (width 0.2) (layer "F.Cu") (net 4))
 (segment (start 177.659193 94.31) (end 176.89 94.31) (width 0.2) (layer "F.Cu") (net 4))
 (segment (start 174.138608 98.48) (end 174.45 98.168608) (width 0.2) (layer "F.Cu") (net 4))
 (segment (start 176.89 94.31) (end 176.55 94.65) (width 0.2) (layer "F.Cu") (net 4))
 (segment (start 177.7 97.1) (end 177.7 96.870001) (width 0.2) (layer "F.Cu") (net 4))
 (via (at 172.8 95.2) (size 0.5) (drill 0.2) (layers "F.Cu" "B.Cu") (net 4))
 (segment (start 173.360589 95.139411) (end 172.860589 95.139411) (width 0.2) (layer "B.Cu") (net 4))
 (segment (start 172.860589 95.139411) (end 172.8 95.2) (width 0.2) (layer "B.Cu") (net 4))
 (segment (start 175.1 98.5) (end 175.1 97.900094) (width 0.2) (layer "F.Cu") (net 16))
 (segment (start 174.949906 97.75) (end 174.8 97.75) (width 0.2) (layer "F.Cu") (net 16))
 (segment (start 174.5 99.1) (end 175.1 98.5) (width 0.2) (layer "F.Cu") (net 16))
 (segment (start 174.1 99.1) (end 174.5 99.1) (width 0.2) (layer "F.Cu") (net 16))
 (segment (start 175.1 97.900094) (end 174.949906 97.75) (width 0.2) (layer "F.Cu") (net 16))
 (via (at 174.1 99.1) (size 0.5) (drill 0.2) (layers "F.Cu" "B.Cu") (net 16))
 (segment (start 174.12 99.5) (end 174.12 99.12) (width 0.2) (layer "B.Cu") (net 16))
 (segment (start 174.12 99.12) (end 174.1 99.1) (width 0.2) (layer "B.Cu") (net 16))
 (segment (start 177.985 95.045929) (end 177.539071 94.6) (width 0.2) (layer "F.Cu") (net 8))
 (segment (start 177.985 95.66) (end 177.985 95.045929) (width 0.2) (layer "F.Cu") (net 8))
 (segment (start 176.9 94.800094) (end 176.9 95.3) (width 0.2) (layer "F.Cu") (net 8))
 (segment (start 177.539071 94.6) (end 177.100094 94.6) (width 0.2) (layer "F.Cu") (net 8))
 (segment (start 177.100094 94.6) (end 176.9 94.800094) (width 0.2) (layer "F.Cu") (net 8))
 (segment (start 178.625 96.3) (end 177.985 95.66) (width 0.2) (layer "F.Cu") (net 8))
 (segment (start 177.985 96.070122) (end 177.695 95.780122) (width 0.2) (layer "F.Cu") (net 6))
 (segment (start 177.985 96.728134) (end 177.985 96.070122) (width 0.2) (layer "F.Cu") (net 6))
 (segment (start 177.5 95.3) (end 177.25 95.3) (width 0.2) (layer "F.Cu") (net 6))
 (segment (start 177.695 95.495) (end 177.5 95.3) (width 0.2) (layer "F.Cu") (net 6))
 (segment (start 178.625 97.368134) (end 177.985 96.728134) (width 0.2) (layer "F.Cu") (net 6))
 (segment (start 178.625 97.4) (end 178.625 97.368134) (width 0.2) (layer "F.Cu") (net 6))
 (segment (start 177.695 95.780122) (end 177.695 95.495) (width 0.2) (layer "F.Cu") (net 6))
 (segment (start 176.5 95.375) (end 176.5 96) (width 0.2) (layer "B.Cu") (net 69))
 (segment (start 177.255 94.62) (end 176.5 95.375) (width 0.2) (layer "B.Cu") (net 69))
 (segment (start 178 98.48) (end 178 97.95) (width 0.2) (layer "B.Cu") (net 75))
 (segment (start 178.9 99.38) (end 178 98.48) (width 0.2) (layer "B.Cu") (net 75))
 (segment (start 175.48 98.12) (end 175.5 98.1) (width 0.2) (layer "F.Cu") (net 5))
 (segment (start 175.48 98.8) (end 175.48 98.12) (width 0.2) (layer "F.Cu") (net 5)))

